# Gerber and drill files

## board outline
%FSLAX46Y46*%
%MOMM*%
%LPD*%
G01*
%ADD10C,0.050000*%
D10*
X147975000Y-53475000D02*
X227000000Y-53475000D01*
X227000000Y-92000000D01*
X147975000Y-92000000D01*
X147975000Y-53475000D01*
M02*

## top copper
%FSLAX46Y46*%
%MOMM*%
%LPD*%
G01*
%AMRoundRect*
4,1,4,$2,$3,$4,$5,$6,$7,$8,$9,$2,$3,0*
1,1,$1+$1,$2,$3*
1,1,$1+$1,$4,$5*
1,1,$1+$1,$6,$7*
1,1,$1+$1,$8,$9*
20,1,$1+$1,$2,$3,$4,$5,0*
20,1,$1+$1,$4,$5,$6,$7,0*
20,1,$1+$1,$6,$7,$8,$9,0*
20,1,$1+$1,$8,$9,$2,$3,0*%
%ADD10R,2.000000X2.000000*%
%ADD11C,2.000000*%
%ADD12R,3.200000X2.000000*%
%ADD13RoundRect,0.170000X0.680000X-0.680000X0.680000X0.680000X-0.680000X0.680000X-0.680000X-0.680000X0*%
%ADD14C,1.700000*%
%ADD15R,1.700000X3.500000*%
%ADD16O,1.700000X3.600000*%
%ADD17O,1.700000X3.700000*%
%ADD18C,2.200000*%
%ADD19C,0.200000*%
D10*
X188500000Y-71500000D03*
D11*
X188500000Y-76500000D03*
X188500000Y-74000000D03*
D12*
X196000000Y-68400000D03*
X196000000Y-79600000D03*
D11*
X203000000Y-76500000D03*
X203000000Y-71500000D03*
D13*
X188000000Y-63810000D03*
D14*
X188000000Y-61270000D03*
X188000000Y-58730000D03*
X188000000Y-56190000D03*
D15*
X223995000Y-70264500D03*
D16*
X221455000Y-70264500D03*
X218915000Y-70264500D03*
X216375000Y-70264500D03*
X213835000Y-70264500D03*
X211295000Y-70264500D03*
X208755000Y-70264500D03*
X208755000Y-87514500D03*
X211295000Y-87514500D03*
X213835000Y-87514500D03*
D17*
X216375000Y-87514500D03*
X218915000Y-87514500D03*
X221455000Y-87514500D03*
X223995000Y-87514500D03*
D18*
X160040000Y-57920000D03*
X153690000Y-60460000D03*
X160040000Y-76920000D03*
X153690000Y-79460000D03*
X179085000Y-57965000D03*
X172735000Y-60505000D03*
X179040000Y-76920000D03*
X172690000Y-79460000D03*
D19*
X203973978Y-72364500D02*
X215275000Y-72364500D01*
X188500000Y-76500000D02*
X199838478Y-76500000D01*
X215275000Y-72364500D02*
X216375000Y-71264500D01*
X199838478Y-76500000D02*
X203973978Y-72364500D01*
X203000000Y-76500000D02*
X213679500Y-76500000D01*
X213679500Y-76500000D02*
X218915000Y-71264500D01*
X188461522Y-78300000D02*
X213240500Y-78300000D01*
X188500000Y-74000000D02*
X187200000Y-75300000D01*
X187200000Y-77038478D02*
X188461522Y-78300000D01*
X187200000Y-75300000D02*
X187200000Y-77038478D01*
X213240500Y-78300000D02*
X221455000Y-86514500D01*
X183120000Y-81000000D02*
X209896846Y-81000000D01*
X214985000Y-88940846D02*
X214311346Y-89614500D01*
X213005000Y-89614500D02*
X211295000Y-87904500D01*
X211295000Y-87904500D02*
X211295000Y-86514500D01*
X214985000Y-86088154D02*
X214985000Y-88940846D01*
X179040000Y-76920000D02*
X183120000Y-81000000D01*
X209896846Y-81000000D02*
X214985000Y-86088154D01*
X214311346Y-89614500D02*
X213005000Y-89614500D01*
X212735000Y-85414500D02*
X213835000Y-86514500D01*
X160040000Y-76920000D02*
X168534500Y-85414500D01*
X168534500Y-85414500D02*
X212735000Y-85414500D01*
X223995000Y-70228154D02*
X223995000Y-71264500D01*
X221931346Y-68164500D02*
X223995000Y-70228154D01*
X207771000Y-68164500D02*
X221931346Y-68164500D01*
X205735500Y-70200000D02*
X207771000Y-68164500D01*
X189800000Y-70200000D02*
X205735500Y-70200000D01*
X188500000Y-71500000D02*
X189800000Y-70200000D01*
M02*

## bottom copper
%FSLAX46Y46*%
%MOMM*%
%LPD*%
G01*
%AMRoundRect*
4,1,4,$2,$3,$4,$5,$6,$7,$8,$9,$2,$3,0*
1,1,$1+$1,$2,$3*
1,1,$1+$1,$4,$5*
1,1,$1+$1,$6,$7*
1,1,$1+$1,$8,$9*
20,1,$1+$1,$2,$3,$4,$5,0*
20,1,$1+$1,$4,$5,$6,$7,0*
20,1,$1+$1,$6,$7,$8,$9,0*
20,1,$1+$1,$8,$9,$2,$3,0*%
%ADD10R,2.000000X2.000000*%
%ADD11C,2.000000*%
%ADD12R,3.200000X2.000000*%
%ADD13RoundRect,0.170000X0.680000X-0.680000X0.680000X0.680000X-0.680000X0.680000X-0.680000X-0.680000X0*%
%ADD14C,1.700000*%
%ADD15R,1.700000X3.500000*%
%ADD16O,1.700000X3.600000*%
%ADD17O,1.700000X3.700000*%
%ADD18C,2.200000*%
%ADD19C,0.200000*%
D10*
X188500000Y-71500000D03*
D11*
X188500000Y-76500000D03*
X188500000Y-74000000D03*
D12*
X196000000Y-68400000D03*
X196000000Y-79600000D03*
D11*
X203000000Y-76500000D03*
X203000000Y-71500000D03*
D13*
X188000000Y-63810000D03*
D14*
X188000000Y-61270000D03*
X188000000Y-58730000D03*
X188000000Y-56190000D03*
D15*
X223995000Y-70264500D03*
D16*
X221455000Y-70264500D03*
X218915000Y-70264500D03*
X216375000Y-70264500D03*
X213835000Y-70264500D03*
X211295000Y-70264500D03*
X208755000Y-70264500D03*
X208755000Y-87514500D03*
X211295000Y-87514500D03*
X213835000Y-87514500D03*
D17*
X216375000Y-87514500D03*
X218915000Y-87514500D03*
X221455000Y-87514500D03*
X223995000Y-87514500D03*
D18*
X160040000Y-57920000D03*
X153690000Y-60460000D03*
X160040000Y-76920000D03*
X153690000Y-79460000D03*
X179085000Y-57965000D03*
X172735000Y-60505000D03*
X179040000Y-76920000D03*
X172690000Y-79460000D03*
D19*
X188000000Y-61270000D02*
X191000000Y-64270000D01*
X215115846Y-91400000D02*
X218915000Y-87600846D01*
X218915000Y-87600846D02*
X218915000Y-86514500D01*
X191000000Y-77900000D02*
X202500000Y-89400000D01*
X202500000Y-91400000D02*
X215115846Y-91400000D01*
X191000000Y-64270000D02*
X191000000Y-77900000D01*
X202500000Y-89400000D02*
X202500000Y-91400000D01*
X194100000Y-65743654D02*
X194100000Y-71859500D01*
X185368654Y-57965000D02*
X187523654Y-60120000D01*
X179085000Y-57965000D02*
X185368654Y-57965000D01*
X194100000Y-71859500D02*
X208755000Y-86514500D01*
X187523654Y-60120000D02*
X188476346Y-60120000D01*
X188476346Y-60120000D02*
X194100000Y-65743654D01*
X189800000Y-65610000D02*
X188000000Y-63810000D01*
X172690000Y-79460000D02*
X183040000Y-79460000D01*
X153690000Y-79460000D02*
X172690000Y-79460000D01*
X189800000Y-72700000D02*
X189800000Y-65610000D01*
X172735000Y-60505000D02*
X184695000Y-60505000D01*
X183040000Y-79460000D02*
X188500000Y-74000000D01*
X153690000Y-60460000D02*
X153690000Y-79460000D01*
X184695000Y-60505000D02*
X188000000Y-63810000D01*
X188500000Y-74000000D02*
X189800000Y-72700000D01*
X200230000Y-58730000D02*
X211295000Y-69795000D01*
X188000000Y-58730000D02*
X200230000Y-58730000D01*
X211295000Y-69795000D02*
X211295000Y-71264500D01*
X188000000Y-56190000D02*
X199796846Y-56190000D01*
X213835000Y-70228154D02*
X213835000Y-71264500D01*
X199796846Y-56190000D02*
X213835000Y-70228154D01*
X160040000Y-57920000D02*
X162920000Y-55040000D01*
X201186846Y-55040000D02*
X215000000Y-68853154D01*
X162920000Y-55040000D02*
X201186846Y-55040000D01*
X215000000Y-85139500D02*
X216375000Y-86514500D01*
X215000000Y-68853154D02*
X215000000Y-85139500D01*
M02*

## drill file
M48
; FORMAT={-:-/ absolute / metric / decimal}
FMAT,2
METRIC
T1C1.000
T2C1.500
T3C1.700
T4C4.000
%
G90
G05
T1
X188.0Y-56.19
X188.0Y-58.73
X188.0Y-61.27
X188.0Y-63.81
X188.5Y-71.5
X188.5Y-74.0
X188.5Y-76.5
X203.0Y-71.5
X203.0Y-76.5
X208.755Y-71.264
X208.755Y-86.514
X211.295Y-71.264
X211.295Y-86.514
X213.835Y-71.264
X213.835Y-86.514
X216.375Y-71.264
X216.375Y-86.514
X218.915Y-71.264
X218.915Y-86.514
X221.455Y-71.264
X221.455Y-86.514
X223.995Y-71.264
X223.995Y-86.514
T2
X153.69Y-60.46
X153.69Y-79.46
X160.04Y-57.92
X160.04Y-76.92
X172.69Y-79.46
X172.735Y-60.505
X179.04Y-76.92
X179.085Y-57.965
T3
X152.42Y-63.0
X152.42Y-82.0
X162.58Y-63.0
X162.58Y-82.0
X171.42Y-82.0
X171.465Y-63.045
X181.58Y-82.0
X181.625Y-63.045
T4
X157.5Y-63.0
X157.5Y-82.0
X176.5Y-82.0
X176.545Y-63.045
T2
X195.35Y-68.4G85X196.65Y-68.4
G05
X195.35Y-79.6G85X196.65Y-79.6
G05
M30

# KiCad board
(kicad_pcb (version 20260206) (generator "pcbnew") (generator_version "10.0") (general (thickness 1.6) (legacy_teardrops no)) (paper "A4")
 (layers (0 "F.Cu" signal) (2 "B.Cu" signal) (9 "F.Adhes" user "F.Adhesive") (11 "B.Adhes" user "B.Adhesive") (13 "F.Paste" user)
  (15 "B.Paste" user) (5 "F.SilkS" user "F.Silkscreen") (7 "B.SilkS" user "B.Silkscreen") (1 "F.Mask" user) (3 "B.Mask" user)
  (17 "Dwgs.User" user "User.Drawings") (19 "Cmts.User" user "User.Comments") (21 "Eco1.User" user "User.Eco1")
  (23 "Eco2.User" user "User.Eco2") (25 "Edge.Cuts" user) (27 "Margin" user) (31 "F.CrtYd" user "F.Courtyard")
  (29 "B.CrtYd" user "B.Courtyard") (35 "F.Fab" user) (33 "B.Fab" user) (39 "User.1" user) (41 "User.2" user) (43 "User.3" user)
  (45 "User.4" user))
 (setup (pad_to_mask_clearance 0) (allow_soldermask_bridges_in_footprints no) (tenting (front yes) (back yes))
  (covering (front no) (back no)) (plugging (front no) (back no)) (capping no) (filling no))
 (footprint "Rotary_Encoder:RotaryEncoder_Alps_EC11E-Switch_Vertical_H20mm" (layer "F.Cu") (at 188.5 71.5)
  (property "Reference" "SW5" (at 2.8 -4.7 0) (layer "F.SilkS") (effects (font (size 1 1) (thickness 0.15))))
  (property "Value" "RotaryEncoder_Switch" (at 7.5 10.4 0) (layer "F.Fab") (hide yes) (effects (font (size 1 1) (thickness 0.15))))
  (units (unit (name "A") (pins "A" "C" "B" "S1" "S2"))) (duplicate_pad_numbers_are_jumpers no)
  (pad "A" thru_hole rect (at 0 0) (size 2 2) (drill 1) (layers "*.Cu" "*.Mask") (remove_unused_layers no) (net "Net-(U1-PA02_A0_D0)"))
  (pad "B" thru_hole circle (at 0 5) (size 2 2) (drill 1) (layers "*.Cu" "*.Mask") (remove_unused_layers no) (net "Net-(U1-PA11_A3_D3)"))
  (pad "C" thru_hole circle (at 0 2.5) (size 2 2) (drill 1) (layers "*.Cu" "*.Mask") (remove_unused_layers no) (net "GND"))
  (pad "MP" thru_hole rect (at 7.5 -3.1) (size 3.2 2) (drill oval 2.8 1.5) (layers "*.Cu" "*.Mask") (remove_unused_layers no))
  (pad "MP" thru_hole rect (at 7.5 8.1) (size 3.2 2) (drill oval 2.8 1.5) (layers "*.Cu" "*.Mask") (remove_unused_layers no))
  (pad "S1" thru_hole circle (at 14.5 5) (size 2 2) (drill 1) (layers "*.Cu" "*.Mask") (remove_unused_layers no) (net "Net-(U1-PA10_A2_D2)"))
  (pad "S2" thru_hole circle (at 14.5 0) (size 2 2) (drill 1) (layers "*.Cu" "*.Mask") (remove_unused_layers no) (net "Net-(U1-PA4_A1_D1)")))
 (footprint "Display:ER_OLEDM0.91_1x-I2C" (layer "F.Cu") (at 188 63.81 90)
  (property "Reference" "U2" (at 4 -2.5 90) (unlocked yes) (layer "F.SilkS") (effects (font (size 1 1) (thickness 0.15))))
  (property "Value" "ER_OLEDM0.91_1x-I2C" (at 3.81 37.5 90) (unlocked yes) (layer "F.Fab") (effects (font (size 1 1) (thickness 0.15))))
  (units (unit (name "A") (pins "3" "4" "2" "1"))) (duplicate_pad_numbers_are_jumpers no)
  (pad "1" thru_hole roundrect (at 0 0 90) (size 1.7 1.7) (drill 1) (layers "*.Cu" "*.Mask") (remove_unused_layers no)
   (roundrect_rratio 0.1) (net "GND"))
  (pad "2" thru_hole circle (at 2.54 0 90) (size 1.7 1.7) (drill 1) (layers "*.Cu" "*.Mask") (remove_unused_layers no) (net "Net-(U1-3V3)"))
  (pad "3" thru_hole circle (at 5.08 0 90) (size 1.7 1.7) (drill 1) (layers "*.Cu" "*.Mask") (remove_unused_layers no)
   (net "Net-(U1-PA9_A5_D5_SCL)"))
  (pad "4" thru_hole circle (at 7.62 0 90) (size 1.7 1.7) (drill 1) (layers "*.Cu" "*.Mask") (remove_unused_layers no)
   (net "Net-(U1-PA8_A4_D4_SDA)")))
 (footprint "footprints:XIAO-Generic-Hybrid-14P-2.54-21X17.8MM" (layer "F.Cu") (at 216.375 78.8895 -90)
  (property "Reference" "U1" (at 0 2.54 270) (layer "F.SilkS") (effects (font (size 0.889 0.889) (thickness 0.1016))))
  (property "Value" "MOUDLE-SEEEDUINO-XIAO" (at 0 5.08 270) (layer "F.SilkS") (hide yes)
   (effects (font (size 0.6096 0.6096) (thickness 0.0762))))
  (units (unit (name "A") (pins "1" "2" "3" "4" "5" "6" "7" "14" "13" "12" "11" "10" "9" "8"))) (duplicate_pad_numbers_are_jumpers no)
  (pad "1" thru_hole rect (at -7.625 -7.62 270) (size 3.5 1.7) (drill 1 (offset -1 0)) (layers "*.Cu" "*.Mask") (remove_unused_layers no)
   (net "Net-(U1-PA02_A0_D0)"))
  (pad "2" thru_hole oval (at -7.625 -5.08 270) (size 3.6 1.7) (drill 1 (offset -1 0)) (layers "*.Cu" "*.Mask") (remove_unused_layers no)
   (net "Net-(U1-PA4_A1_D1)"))
  (pad "3" thru_hole oval (at -7.625 -2.54 270) (size 3.6 1.7) (drill 1 (offset -1 0)) (layers "*.Cu" "*.Mask") (remove_unused_layers no)
   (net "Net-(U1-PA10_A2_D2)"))
  (pad "4" thru_hole oval (at -7.625 0 270) (size 3.6 1.7) (drill 1 (offset -1 0)) (layers "*.Cu" "*.Mask") (remove_unused_layers no)
   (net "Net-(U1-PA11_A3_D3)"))
  (pad "5" thru_hole oval (at -7.625 2.54 270) (size 3.6 1.7) (drill 1 (offset -1 0)) (layers "*.Cu" "*.Mask") (remove_unused_layers no)
   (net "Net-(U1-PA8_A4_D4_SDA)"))
  (pad "6" thru_hole oval (at -7.625 5.08 90) (size 3.6 1.7) (drill 1 (offset 1 0)) (layers "*.Cu" "*.Mask") (remove_unused_layers no)
   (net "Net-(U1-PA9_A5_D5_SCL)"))
  (pad "7" thru_hole oval (at -7.625 7.62 270) (size 3.6 1.7) (drill 1 (offset -1 0)) (layers "*.Cu" "*.Mask") (remove_unused_layers no)
   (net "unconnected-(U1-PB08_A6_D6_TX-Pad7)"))
  (pad "8" thru_hole oval (at 7.625 7.62 270) (size 3.6 1.7) (drill 1 (offset 1 0)) (layers "*.Cu" "*.Mask") (remove_unused_layers no)
   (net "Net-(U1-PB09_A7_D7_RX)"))
  (pad "9" thru_hole oval (at 7.625 5.08 270) (size 3.6 1.7) (drill 1 (offset 1 0)) (layers "*.Cu" "*.Mask") (remove_unused_layers no)
   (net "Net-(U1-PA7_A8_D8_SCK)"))
  (pad "10" thru_hole oval (at 7.625 2.54 270) (size 3.6 1.7) (drill 1 (offset 1 0)) (layers "*.Cu" "*.Mask") (remove_unused_layers no)
   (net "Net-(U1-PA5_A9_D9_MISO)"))
  (pad "11" thru_hole oval (at 7.625 0 270) (size 3.7 1.7) (drill 1 (offset 1 0)) (layers "*.Cu" "*.Mask") (remove_unused_layers no)
   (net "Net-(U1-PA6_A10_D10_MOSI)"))
  (pad "12" thru_hole oval (at 7.625 -2.54 270) (size 3.7 1.7) (drill 1 (offset 1 0)) (layers "*.Cu" "*.Mask") (remove_unused_layers no)
   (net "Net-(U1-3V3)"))
  (pad "13" thru_hole oval (at 7.625 -5.08 270) (size 3.7 1.7) (drill 1 (offset 1 0)) (layers "*.Cu" "*.Mask") (remove_unused_layers no)
   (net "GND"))
  (pad "14" thru_hole oval (at 7.625 -7.62 270) (size 3.7 1.7) (drill 1 (offset 1 0)) (layers "*.Cu" "*.Mask") (remove_unused_layers no)
   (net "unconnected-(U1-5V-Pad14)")))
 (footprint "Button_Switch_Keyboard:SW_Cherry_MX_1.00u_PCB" (layer "F.Cu") (at 160.04 57.92)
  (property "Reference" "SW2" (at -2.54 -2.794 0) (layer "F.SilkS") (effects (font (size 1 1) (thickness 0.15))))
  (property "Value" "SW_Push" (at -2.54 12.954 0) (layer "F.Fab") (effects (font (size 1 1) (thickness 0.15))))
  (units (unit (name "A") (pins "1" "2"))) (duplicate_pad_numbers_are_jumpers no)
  (pad "" np_thru_hole circle (at -7.62 5.08) (size 1.7 1.7) (drill 1.7) (layers "*.Cu" "*.Mask"))
  (pad "" np_thru_hole circle (at -2.54 5.08) (size 4 4) (drill 4) (layers "*.Cu" "*.Mask"))
  (pad "" np_thru_hole circle (at 2.54 5.08) (size 1.7 1.7) (drill 1.7) (layers "*.Cu" "*.Mask"))
  (pad "1" thru_hole circle (at 0 0) (size 2.2 2.2) (drill 1.5) (layers "*.Cu" "*.Mask") (remove_unused_layers no)
   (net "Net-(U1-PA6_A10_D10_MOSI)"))
  (pad "2" thru_hole circle (at -6.35 2.54) (size 2.2 2.2) (drill 1.5) (layers "*.Cu" "*.Mask") (remove_unused_layers no) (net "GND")))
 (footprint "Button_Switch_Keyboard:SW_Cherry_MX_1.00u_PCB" (layer "F.Cu") (at 160.04 76.92)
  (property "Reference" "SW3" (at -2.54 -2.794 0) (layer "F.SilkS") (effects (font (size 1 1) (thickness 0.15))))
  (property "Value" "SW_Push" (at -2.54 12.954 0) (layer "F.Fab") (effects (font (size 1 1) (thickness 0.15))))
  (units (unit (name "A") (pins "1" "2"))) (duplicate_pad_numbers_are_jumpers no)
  (pad "" np_thru_hole circle (at -7.62 5.08) (size 1.7 1.7) (drill 1.7) (layers "*.Cu" "*.Mask"))
  (pad "" np_thru_hole circle (at -2.54 5.08) (size 4 4) (drill 4) (layers "*.Cu" "*.Mask"))
  (pad "" np_thru_hole circle (at 2.54 5.08) (size 1.7 1.7) (drill 1.7) (layers "*.Cu" "*.Mask"))
  (pad "1" thru_hole circle (at 0 0) (size 2.2 2.2) (drill 1.5) (layers "*.Cu" "*.Mask") (remove_unused_layers no)
   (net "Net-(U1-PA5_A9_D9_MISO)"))
  (pad "2" thru_hole circle (at -6.35 2.54) (size 2.2 2.2) (drill 1.5) (layers "*.Cu" "*.Mask") (remove_unused_layers no) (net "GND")))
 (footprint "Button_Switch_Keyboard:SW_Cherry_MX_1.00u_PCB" (layer "F.Cu") (at 179.085 57.965)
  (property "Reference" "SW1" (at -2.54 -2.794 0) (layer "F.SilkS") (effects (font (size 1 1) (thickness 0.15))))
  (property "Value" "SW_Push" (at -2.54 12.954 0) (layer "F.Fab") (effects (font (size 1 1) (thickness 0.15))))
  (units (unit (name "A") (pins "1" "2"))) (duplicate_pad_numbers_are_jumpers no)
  (pad "" np_thru_hole circle (at -7.62 5.08) (size 1.7 1.7) (drill 1.7) (layers "*.Cu" "*.Mask"))
  (pad "" np_thru_hole circle (at -2.54 5.08) (size 4 4) (drill 4) (layers "*.Cu" "*.Mask"))
  (pad "" np_thru_hole circle (at 2.54 5.08) (size 1.7 1.7) (drill 1.7) (layers "*.Cu" "*.Mask"))
  (pad "1" thru_hole circle (at 0 0) (size 2.2 2.2) (drill 1.5) (layers "*.Cu" "*.Mask") (remove_unused_layers no)
   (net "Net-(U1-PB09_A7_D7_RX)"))
  (pad "2" thru_hole circle (at -6.35 2.54) (size 2.2 2.2) (drill 1.5) (layers "*.Cu" "*.Mask") (remove_unused_layers no) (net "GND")))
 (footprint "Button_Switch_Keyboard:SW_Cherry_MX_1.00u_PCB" (layer "F.Cu") (at 179.04 76.92)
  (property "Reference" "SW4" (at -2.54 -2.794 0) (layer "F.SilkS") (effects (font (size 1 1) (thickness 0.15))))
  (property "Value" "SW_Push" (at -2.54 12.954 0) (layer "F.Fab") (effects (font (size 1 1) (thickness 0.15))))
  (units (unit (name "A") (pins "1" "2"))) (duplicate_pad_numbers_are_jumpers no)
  (pad "" np_thru_hole circle (at -7.62 5.08) (size 1.7 1.7) (drill 1.7) (layers "*.Cu" "*.Mask"))
  (pad "" np_thru_hole circle (at -2.54 5.08) (size 4 4) (drill 4) (layers "*.Cu" "*.Mask"))
  (pad "" np_thru_hole circle (at 2.54 5.08) (size 1.7 1.7) (drill 1.7) (layers "*.Cu" "*.Mask"))
  (pad "1" thru_hole circle (at 0 0) (size 2.2 2.2) (drill 1.5) (layers "*.Cu" "*.Mask") (remove_unused_layers no)
   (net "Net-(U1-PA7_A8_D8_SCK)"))
  (pad "2" thru_hole circle (at -6.35 2.54) (size 2.2 2.2) (drill 1.5) (layers "*.Cu" "*.Mask") (remove_unused_layers no) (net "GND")))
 (gr_rect (start 147.975 53.475) (end 227 92) (stroke (width 0.05) (type default)) (fill no) (layer "Edge.Cuts"))
 (segment (start 188 61.27) (end 191 64.27) (width 0.2) (layer "B.Cu") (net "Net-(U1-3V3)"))
 (segment (start 215.115846 91.4) (end 218.915 87.600846) (width 0.2) (layer "B.Cu") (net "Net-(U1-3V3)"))
 (segment (start 218.915 87.600846) (end 218.915 86.5145) (width 0.2) (layer "B.Cu") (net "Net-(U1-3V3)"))
 (segment (start 191 77.9) (end 202.5 89.4) (width 0.2) (layer "B.Cu") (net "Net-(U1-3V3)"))
 (segment (start 202.5 91.4) (end 215.115846 91.4) (width 0.2) (layer "B.Cu") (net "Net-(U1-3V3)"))
 (segment (start 191 64.27) (end 191 77.9) (width 0.2) (layer "B.Cu") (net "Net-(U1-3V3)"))
 (segment (start 202.5 89.4) (end 202.5 91.4) (width 0.2) (layer "B.Cu") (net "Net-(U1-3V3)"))
 (segment (start 194.1 65.743654) (end 194.1 71.8595) (width 0.2) (layer "B.Cu") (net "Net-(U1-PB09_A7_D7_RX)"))
 (segment (start 185.368654 57.965) (end 187.523654 60.12) (width 0.2) (layer "B.Cu") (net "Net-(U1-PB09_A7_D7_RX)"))
 (segment (start 179.085 57.965) (end 185.368654 57.965) (width 0.2) (layer "B.Cu") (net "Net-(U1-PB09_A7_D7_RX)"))
 (segment (start 194.1 71.8595) (end 208.755 86.5145) (width 0.2) (layer "B.Cu") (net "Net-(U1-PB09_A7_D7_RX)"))
 (segment (start 187.523654 60.12) (end 188.476346 60.12) (width 0.2) (layer "B.Cu") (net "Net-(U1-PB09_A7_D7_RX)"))
 (segment (start 188.476346 60.12) (end 194.1 65.743654) (width 0.2) (layer "B.Cu") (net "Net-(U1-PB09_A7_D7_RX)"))
 (segment (start 203.973978 72.3645) (end 215.275 72.3645) (width 0.2) (layer "F.Cu") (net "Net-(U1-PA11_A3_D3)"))
 (segment (start 188.5 76.5) (end 199.838478 76.5) (width 0.2) (layer "F.Cu") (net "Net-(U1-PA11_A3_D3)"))
 (segment (start 215.275 72.3645) (end 216.375 71.2645) (width 0.2) (layer "F.Cu") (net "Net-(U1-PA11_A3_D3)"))
 (segment (start 199.838478 76.5) (end 203.973978 72.3645) (width 0.2) (layer "F.Cu") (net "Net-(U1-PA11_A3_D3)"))
 (segment (start 203 76.5) (end 213.6795 76.5) (width 0.2) (layer "F.Cu") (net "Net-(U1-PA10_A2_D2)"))
 (segment (start 213.6795 76.5) (end 218.915 71.2645) (width 0.2) (layer "F.Cu") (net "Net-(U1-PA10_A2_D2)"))
 (segment (start 188.461522 78.3) (end 213.2405 78.3) (width 0.2) (layer "F.Cu") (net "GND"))
 (segment (start 188.5 74) (end 187.2 75.3) (width 0.2) (layer "F.Cu") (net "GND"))
 (segment (start 187.2 77.038478) (end 188.461522 78.3) (width 0.2) (layer "F.Cu") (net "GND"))
 (segment (start 187.2 75.3) (end 187.2 77.038478) (width 0.2) (layer "F.Cu") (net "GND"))
 (segment (start 213.2405 78.3) (end 221.455 86.5145) (width 0.2) (layer "F.Cu") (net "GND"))
 (segment (start 189.8 65.61) (end 188 63.81) (width 0.2) (layer "B.Cu") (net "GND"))
 (segment (start 172.69 79.46) (end 183.04 79.46) (width 0.2) (layer "B.Cu") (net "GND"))
 (segment (start 153.69 79.46) (end 172.69 79.46) (width 0.2) (layer "B.Cu") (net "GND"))
 (segment (start 189.8 72.7) (end 189.8 65.61) (width 0.2) (layer "B.Cu") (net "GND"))
 (segment (start 172.735 60.505) (end 184.695 60.505) (width 0.2) (layer "B.Cu") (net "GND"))
 (segment (start 183.04 79.46) (end 188.5 74) (width 0.2) (layer "B.Cu") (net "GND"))
 (segment (start 153.69 60.46) (end 153.69 79.46) (width 0.2) (layer "B.Cu") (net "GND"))
 (segment (start 184.695 60.505) (end 188 63.81) (width 0.2) (layer "B.Cu") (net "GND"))
 (segment (start 188.5 74) (end 189.8 72.7) (width 0.2) (layer "B.Cu") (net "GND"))
 (segment (start 200.23 58.73) (end 211.295 69.795) (width 0.2) (layer "B.Cu") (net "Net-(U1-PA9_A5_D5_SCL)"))
 (segment (start 188 58.73) (end 200.23 58.73) (width 0.2) (layer "B.Cu") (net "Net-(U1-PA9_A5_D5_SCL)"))
 (segment (start 211.295 69.795) (end 211.295 71.2645) (width 0.2) (layer "B.Cu") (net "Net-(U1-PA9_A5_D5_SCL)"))
 (segment (start 188 56.19) (end 199.796846 56.19) (width 0.2) (layer "B.Cu") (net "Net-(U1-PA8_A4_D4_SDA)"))
 (segment (start 213.835 70.228154) (end 213.835 71.2645) (width 0.2) (layer "B.Cu") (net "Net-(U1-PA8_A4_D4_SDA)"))
 (segment (start 199.796846 56.19) (end 213.835 70.228154) (width 0.2) (layer "B.Cu") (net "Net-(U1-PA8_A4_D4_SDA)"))
 (segment (start 183.12 81) (end 209.896846 81) (width 0.2) (layer "F.Cu") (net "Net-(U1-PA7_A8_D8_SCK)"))
 (segment (start 214.985 88.940846) (end 214.311346 89.6145) (width 0.2) (layer "F.Cu") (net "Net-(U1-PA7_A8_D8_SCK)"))
 (segment (start 213.005 89.6145) (end 211.295 87.9045) (width 0.2) (layer "F.Cu") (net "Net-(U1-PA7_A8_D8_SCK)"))
 (segment (start 211.295 87.9045) (end 211.295 86.5145) (width 0.2) (layer "F.Cu") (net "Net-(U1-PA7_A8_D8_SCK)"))
 (segment (start 214.985 86.088154) (end 214.985 88.940846) (width 0.2) (layer "F.Cu") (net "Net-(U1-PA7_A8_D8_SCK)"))
 (segment (start 179.04 76.92) (end 183.12 81) (width 0.2) (layer "F.Cu") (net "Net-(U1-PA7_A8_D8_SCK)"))
 (segment (start 209.896846 81) (end 214.985 86.088154) (width 0.2) (layer "F.Cu") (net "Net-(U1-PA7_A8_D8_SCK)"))
 (segment (start 214.311346 89.6145) (end 213.005 89.6145) (width 0.2) (layer "F.Cu") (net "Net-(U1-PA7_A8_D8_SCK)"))
 (segment (start 212.735 85.4145) (end 213.835 86.5145) (width 0.2) (layer "F.Cu") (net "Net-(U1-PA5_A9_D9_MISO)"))
 (segment (start 160.04 76.92) (end 168.5345 85.4145) (width 0.2) (layer "F.Cu") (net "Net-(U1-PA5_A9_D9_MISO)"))
 (segment (start 168.5345 85.4145) (end 212.735 85.4145) (width 0.2) (layer "F.Cu") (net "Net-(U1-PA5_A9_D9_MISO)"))
 (segment (start 160.04 57.92) (end 162.92 55.04) (width 0.2) (layer "B.Cu") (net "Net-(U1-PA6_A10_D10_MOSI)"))
 (segment (start 201.186846 55.04) (end 215 68.853154) (width 0.2) (layer "B.Cu") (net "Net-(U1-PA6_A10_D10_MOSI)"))
 (segment (start 162.92 55.04) (end 201.186846 55.04) (width 0.2) (layer "B.Cu") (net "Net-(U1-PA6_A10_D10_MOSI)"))
 (segment (start 215 85.1395) (end 216.375 86.5145) (width 0.2) (layer "B.Cu") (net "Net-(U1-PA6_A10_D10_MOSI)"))
 (segment (start 215 68.853154) (end 215 85.1395) (width 0.2) (layer "B.Cu") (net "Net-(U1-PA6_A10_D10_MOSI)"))
 (segment (start 223.995 70.228154) (end 223.995 71.2645) (width 0.2) (layer "F.Cu") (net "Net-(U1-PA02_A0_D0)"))
 (segment (start 221.931346 68.1645) (end 223.995 70.228154) (width 0.2) (layer "F.Cu") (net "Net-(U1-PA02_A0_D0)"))
 (segment (start 207.771 68.1645) (end 221.931346 68.1645) (width 0.2) (layer "F.Cu") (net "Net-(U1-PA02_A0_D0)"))
 (segment (start 205.7355 70.2) (end 207.771 68.1645) (width 0.2) (layer "F.Cu") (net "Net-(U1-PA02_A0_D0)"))
 (segment (start 189.8 70.2) (end 205.7355 70.2) (width 0.2) (layer "F.Cu") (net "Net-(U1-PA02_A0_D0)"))
 (segment (start 188.5 71.5) (end 189.8 70.2) (width 0.2) (layer "F.Cu") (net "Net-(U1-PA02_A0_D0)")))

